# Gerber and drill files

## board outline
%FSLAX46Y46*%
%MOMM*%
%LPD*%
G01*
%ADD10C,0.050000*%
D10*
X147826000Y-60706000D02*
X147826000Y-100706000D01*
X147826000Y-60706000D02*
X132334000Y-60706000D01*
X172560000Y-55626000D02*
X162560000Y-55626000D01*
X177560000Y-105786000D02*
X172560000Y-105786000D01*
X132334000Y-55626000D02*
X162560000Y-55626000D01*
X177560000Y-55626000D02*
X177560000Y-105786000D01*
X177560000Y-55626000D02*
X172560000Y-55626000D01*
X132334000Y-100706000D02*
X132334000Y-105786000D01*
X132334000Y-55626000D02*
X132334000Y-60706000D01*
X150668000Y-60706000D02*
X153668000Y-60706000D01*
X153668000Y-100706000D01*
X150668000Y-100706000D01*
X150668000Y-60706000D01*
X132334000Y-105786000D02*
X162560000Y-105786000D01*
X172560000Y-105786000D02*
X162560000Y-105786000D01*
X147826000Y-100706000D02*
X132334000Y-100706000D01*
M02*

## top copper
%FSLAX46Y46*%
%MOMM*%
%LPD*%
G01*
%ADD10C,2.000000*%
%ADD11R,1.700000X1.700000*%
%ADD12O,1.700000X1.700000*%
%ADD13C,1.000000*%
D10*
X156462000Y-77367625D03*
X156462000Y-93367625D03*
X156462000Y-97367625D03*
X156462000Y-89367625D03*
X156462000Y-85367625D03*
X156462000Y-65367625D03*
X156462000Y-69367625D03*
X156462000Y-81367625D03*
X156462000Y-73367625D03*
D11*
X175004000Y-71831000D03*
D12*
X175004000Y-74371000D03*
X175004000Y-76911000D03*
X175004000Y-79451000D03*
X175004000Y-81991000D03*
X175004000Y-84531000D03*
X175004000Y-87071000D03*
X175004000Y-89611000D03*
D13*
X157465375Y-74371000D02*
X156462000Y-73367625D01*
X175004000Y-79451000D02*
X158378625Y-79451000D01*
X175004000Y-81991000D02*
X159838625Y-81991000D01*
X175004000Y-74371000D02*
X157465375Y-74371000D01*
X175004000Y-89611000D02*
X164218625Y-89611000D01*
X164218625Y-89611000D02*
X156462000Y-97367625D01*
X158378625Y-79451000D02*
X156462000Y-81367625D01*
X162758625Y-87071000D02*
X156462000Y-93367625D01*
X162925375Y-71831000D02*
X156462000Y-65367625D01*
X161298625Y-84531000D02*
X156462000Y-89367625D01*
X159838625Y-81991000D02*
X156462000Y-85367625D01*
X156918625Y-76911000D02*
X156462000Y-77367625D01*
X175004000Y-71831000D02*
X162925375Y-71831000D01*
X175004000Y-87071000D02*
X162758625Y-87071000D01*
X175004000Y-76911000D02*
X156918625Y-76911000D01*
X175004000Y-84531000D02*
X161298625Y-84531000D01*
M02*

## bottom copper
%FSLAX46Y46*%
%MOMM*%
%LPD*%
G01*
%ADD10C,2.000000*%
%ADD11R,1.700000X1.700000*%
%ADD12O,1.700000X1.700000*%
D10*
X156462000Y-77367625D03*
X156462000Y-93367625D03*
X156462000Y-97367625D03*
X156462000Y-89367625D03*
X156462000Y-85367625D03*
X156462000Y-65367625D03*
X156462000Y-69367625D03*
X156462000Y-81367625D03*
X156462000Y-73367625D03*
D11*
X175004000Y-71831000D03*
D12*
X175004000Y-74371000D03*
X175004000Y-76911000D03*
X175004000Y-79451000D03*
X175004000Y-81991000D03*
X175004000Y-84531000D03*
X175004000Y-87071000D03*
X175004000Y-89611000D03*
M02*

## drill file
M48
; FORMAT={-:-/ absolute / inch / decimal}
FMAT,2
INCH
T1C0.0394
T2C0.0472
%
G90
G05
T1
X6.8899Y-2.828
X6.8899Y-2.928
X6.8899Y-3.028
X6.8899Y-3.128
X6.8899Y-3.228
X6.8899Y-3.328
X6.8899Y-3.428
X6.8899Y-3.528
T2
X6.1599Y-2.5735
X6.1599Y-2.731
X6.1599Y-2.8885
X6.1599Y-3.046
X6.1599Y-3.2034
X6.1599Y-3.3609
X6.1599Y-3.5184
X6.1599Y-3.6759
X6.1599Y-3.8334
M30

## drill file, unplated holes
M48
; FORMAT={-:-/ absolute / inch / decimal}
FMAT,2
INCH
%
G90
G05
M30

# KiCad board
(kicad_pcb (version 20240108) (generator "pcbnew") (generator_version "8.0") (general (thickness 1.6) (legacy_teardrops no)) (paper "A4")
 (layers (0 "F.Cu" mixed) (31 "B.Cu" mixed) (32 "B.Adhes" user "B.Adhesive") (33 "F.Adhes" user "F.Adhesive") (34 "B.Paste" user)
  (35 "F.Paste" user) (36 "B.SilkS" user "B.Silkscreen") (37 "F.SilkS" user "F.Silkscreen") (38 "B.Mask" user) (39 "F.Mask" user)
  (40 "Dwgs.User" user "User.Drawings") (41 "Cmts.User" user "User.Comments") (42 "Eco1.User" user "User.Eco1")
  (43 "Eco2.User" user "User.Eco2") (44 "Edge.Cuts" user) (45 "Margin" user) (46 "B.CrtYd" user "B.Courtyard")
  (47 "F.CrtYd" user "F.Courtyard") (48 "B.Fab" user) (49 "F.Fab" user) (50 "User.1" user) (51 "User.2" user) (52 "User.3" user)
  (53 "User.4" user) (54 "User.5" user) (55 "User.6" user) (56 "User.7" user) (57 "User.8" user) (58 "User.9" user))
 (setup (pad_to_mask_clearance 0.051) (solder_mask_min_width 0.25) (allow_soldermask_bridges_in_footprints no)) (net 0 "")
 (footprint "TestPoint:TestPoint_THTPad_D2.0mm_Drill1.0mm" (layer "F.Cu") (at 156.462 77.367625)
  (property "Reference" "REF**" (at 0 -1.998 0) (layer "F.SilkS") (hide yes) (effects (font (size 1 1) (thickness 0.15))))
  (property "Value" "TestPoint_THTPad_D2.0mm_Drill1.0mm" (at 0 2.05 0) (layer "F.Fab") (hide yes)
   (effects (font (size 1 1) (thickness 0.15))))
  (pad "6" thru_hole circle (at 0 0) (size 2 2) (drill 1.2) (layers "*.Cu" "*.Mask") (remove_unused_layers no)))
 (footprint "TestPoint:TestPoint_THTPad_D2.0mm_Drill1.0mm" (layer "F.Cu") (at 156.462 93.367625)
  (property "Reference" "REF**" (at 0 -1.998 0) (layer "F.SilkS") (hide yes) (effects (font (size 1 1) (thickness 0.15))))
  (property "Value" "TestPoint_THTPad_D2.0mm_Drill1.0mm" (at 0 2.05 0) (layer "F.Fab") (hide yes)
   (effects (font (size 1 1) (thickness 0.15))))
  (pad "2" thru_hole circle (at 0 0) (size 2 2) (drill 1.2) (layers "*.Cu" "*.Mask") (remove_unused_layers no)))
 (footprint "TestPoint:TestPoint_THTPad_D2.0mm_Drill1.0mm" (layer "F.Cu") (at 156.462 97.367625)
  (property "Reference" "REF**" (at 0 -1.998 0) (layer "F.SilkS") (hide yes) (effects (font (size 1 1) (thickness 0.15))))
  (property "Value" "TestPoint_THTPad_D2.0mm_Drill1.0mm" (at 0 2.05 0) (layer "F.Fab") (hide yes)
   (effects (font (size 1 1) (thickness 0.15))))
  (pad "1" thru_hole circle (at 0 0) (size 2 2) (drill 1.2) (layers "*.Cu" "*.Mask") (remove_unused_layers no)))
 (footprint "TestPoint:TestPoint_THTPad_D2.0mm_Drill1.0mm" (layer "F.Cu") (at 156.462 89.367625)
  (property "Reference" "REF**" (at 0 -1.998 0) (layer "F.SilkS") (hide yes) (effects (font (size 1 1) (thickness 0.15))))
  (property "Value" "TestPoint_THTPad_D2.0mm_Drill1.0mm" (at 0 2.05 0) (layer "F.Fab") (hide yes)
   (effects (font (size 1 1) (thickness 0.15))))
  (pad "3" thru_hole circle (at 0 0) (size 2 2) (drill 1.2) (layers "*.Cu" "*.Mask") (remove_unused_layers no)))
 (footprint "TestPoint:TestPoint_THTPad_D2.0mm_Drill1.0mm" (layer "F.Cu") (at 156.462 85.367625)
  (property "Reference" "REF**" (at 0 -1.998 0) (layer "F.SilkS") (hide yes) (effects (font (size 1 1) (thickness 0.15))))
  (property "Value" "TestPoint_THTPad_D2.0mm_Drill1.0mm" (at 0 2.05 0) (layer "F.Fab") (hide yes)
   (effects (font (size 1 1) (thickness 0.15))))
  (pad "4" thru_hole circle (at 0 0) (size 2 2) (drill 1.2) (layers "*.Cu" "*.Mask") (remove_unused_layers no)))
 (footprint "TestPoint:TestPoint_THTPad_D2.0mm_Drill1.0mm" (layer "F.Cu") (at 156.462 65.367625)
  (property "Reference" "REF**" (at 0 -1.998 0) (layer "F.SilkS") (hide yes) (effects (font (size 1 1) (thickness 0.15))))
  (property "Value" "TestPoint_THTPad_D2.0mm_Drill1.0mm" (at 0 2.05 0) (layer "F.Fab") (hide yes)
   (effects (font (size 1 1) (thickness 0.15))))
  (pad "9" thru_hole circle (at 0 0) (size 2 2) (drill 1.2) (layers "*.Cu" "*.Mask") (remove_unused_layers no)))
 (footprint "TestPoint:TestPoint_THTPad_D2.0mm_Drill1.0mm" (layer "F.Cu") (at 156.462 69.367625)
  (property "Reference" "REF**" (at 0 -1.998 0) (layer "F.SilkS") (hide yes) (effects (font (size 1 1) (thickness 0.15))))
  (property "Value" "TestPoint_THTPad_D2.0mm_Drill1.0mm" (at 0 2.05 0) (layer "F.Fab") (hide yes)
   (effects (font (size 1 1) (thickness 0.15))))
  (pad "8" thru_hole circle (at 0 0) (size 2 2) (drill 1.2) (layers "*.Cu" "*.Mask") (remove_unused_layers no)))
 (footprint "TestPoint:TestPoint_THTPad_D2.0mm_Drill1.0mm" (layer "F.Cu") (at 156.462 81.367625)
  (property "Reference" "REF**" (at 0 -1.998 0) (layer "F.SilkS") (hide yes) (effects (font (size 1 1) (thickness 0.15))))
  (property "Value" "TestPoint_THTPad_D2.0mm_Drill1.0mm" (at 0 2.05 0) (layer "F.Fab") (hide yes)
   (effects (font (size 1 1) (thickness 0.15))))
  (pad "5" thru_hole circle (at 0 0) (size 2 2) (drill 1.2) (layers "*.Cu" "*.Mask") (remove_unused_layers no)))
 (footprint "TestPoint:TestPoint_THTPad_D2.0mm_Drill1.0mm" (layer "F.Cu") (at 156.462 73.367625)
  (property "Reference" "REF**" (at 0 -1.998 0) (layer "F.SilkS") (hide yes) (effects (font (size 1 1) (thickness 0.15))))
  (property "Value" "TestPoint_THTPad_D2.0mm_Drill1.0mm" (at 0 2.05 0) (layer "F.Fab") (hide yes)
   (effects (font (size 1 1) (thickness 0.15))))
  (pad "7" thru_hole circle (at 0 0) (size 2 2) (drill 1.2) (layers "*.Cu" "*.Mask") (remove_unused_layers no)))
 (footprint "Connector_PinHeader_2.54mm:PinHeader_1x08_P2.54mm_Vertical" (layer "F.Cu") (at 175.004 71.831)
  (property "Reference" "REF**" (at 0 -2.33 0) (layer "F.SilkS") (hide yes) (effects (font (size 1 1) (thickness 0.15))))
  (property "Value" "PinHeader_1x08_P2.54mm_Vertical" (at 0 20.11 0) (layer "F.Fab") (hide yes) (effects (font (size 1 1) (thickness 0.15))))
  (pad "1" thru_hole rect (at 0 0) (size 1.7 1.7) (drill 1) (layers "*.Cu" "*.Mask") (remove_unused_layers no))
  (pad "2" thru_hole oval (at 0 2.54) (size 1.7 1.7) (drill 1) (layers "*.Cu" "*.Mask") (remove_unused_layers no))
  (pad "3" thru_hole oval (at 0 5.08) (size 1.7 1.7) (drill 1) (layers "*.Cu" "*.Mask") (remove_unused_layers no))
  (pad "4" thru_hole oval (at 0 7.62) (size 1.7 1.7) (drill 1) (layers "*.Cu" "*.Mask") (remove_unused_layers no))
  (pad "5" thru_hole oval (at 0 10.16) (size 1.7 1.7) (drill 1) (layers "*.Cu" "*.Mask") (remove_unused_layers no))
  (pad "6" thru_hole oval (at 0 12.7) (size 1.7 1.7) (drill 1) (layers "*.Cu" "*.Mask") (remove_unused_layers no))
  (pad "7" thru_hole oval (at 0 15.24) (size 1.7 1.7) (drill 1) (layers "*.Cu" "*.Mask") (remove_unused_layers no))
  (pad "8" thru_hole oval (at 0 17.78) (size 1.7 1.7) (drill 1) (layers "*.Cu" "*.Mask") (remove_unused_layers no)))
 (gr_line (start 147.826 60.706) (end 147.826 100.706) (stroke (width 0.05) (type default)) (layer "Edge.Cuts"))
 (gr_line (start 147.826 60.706) (end 132.334 60.706) (stroke (width 0.05) (type default)) (layer "Edge.Cuts"))
 (gr_line (start 172.56 55.626) (end 162.56 55.626) (stroke (width 0.05) (type default)) (layer "Edge.Cuts"))
 (gr_line (start 177.56 105.786) (end 172.56 105.786) (stroke (width 0.05) (type default)) (layer "Edge.Cuts"))
 (gr_line (start 132.334 55.626) (end 162.56 55.626) (stroke (width 0.05) (type default)) (layer "Edge.Cuts"))
 (gr_line (start 177.56 55.626) (end 177.56 105.786) (stroke (width 0.05) (type default)) (layer "Edge.Cuts"))
 (gr_line (start 177.56 55.626) (end 172.56 55.626) (stroke (width 0.05) (type default)) (layer "Edge.Cuts"))
 (gr_line (start 132.334 100.706) (end 132.334 105.786) (stroke (width 0.05) (type default)) (layer "Edge.Cuts"))
 (gr_line (start 132.334 55.626) (end 132.334 60.706) (stroke (width 0.05) (type default)) (layer "Edge.Cuts"))
 (gr_rect (start 150.668 60.706) (end 153.668 100.706) (stroke (width 0.05) (type default)) (fill none) (layer "Edge.Cuts"))
 (gr_line (start 132.334 105.786) (end 162.56 105.786) (stroke (width 0.05) (type default)) (layer "Edge.Cuts"))
 (gr_line (start 172.56 105.786) (end 162.56 105.786) (stroke (width 0.05) (type default)) (layer "Edge.Cuts"))
 (gr_line (start 147.826 100.706) (end 132.334 100.706) (stroke (width 0.05) (type default)) (layer "Edge.Cuts"))
 (segment (start 157.465375 74.371) (end 156.462 73.367625) (width 1) (layer "F.Cu") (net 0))
 (segment (start 175.004 79.451) (end 158.378625 79.451) (width 1) (layer "F.Cu") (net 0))
 (segment (start 175.004 81.991) (end 159.838625 81.991) (width 1) (layer "F.Cu") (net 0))
 (segment (start 175.004 74.371) (end 157.465375 74.371) (width 1) (layer "F.Cu") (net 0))
 (segment (start 175.004 89.611) (end 164.218625 89.611) (width 1) (layer "F.Cu") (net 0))
 (segment (start 164.218625 89.611) (end 156.462 97.367625) (width 1) (layer "F.Cu") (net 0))
 (segment (start 158.378625 79.451) (end 156.462 81.367625) (width 1) (layer "F.Cu") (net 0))
 (segment (start 162.758625 87.071) (end 156.462 93.367625) (width 1) (layer "F.Cu") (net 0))
 (segment (start 162.925375 71.831) (end 156.462 65.367625) (width 1) (layer "F.Cu") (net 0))
 (segment (start 161.298625 84.531) (end 156.462 89.367625) (width 1) (layer "F.Cu") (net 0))
 (segment (start 159.838625 81.991) (end 156.462 85.367625) (width 1) (layer "F.Cu") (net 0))
 (segment (start 156.918625 76.911) (end 156.462 77.367625) (width 1) (layer "F.Cu") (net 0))
 (segment (start 175.004 71.831) (end 162.925375 71.831) (width 1) (layer "F.Cu") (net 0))
 (segment (start 175.004 87.071) (end 162.758625 87.071) (width 1) (layer "F.Cu") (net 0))
 (segment (start 175.004 76.911) (end 156.918625 76.911) (width 1) (layer "F.Cu") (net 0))
 (segment (start 175.004 84.531) (end 161.298625 84.531) (width 1) (layer "F.Cu") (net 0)))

